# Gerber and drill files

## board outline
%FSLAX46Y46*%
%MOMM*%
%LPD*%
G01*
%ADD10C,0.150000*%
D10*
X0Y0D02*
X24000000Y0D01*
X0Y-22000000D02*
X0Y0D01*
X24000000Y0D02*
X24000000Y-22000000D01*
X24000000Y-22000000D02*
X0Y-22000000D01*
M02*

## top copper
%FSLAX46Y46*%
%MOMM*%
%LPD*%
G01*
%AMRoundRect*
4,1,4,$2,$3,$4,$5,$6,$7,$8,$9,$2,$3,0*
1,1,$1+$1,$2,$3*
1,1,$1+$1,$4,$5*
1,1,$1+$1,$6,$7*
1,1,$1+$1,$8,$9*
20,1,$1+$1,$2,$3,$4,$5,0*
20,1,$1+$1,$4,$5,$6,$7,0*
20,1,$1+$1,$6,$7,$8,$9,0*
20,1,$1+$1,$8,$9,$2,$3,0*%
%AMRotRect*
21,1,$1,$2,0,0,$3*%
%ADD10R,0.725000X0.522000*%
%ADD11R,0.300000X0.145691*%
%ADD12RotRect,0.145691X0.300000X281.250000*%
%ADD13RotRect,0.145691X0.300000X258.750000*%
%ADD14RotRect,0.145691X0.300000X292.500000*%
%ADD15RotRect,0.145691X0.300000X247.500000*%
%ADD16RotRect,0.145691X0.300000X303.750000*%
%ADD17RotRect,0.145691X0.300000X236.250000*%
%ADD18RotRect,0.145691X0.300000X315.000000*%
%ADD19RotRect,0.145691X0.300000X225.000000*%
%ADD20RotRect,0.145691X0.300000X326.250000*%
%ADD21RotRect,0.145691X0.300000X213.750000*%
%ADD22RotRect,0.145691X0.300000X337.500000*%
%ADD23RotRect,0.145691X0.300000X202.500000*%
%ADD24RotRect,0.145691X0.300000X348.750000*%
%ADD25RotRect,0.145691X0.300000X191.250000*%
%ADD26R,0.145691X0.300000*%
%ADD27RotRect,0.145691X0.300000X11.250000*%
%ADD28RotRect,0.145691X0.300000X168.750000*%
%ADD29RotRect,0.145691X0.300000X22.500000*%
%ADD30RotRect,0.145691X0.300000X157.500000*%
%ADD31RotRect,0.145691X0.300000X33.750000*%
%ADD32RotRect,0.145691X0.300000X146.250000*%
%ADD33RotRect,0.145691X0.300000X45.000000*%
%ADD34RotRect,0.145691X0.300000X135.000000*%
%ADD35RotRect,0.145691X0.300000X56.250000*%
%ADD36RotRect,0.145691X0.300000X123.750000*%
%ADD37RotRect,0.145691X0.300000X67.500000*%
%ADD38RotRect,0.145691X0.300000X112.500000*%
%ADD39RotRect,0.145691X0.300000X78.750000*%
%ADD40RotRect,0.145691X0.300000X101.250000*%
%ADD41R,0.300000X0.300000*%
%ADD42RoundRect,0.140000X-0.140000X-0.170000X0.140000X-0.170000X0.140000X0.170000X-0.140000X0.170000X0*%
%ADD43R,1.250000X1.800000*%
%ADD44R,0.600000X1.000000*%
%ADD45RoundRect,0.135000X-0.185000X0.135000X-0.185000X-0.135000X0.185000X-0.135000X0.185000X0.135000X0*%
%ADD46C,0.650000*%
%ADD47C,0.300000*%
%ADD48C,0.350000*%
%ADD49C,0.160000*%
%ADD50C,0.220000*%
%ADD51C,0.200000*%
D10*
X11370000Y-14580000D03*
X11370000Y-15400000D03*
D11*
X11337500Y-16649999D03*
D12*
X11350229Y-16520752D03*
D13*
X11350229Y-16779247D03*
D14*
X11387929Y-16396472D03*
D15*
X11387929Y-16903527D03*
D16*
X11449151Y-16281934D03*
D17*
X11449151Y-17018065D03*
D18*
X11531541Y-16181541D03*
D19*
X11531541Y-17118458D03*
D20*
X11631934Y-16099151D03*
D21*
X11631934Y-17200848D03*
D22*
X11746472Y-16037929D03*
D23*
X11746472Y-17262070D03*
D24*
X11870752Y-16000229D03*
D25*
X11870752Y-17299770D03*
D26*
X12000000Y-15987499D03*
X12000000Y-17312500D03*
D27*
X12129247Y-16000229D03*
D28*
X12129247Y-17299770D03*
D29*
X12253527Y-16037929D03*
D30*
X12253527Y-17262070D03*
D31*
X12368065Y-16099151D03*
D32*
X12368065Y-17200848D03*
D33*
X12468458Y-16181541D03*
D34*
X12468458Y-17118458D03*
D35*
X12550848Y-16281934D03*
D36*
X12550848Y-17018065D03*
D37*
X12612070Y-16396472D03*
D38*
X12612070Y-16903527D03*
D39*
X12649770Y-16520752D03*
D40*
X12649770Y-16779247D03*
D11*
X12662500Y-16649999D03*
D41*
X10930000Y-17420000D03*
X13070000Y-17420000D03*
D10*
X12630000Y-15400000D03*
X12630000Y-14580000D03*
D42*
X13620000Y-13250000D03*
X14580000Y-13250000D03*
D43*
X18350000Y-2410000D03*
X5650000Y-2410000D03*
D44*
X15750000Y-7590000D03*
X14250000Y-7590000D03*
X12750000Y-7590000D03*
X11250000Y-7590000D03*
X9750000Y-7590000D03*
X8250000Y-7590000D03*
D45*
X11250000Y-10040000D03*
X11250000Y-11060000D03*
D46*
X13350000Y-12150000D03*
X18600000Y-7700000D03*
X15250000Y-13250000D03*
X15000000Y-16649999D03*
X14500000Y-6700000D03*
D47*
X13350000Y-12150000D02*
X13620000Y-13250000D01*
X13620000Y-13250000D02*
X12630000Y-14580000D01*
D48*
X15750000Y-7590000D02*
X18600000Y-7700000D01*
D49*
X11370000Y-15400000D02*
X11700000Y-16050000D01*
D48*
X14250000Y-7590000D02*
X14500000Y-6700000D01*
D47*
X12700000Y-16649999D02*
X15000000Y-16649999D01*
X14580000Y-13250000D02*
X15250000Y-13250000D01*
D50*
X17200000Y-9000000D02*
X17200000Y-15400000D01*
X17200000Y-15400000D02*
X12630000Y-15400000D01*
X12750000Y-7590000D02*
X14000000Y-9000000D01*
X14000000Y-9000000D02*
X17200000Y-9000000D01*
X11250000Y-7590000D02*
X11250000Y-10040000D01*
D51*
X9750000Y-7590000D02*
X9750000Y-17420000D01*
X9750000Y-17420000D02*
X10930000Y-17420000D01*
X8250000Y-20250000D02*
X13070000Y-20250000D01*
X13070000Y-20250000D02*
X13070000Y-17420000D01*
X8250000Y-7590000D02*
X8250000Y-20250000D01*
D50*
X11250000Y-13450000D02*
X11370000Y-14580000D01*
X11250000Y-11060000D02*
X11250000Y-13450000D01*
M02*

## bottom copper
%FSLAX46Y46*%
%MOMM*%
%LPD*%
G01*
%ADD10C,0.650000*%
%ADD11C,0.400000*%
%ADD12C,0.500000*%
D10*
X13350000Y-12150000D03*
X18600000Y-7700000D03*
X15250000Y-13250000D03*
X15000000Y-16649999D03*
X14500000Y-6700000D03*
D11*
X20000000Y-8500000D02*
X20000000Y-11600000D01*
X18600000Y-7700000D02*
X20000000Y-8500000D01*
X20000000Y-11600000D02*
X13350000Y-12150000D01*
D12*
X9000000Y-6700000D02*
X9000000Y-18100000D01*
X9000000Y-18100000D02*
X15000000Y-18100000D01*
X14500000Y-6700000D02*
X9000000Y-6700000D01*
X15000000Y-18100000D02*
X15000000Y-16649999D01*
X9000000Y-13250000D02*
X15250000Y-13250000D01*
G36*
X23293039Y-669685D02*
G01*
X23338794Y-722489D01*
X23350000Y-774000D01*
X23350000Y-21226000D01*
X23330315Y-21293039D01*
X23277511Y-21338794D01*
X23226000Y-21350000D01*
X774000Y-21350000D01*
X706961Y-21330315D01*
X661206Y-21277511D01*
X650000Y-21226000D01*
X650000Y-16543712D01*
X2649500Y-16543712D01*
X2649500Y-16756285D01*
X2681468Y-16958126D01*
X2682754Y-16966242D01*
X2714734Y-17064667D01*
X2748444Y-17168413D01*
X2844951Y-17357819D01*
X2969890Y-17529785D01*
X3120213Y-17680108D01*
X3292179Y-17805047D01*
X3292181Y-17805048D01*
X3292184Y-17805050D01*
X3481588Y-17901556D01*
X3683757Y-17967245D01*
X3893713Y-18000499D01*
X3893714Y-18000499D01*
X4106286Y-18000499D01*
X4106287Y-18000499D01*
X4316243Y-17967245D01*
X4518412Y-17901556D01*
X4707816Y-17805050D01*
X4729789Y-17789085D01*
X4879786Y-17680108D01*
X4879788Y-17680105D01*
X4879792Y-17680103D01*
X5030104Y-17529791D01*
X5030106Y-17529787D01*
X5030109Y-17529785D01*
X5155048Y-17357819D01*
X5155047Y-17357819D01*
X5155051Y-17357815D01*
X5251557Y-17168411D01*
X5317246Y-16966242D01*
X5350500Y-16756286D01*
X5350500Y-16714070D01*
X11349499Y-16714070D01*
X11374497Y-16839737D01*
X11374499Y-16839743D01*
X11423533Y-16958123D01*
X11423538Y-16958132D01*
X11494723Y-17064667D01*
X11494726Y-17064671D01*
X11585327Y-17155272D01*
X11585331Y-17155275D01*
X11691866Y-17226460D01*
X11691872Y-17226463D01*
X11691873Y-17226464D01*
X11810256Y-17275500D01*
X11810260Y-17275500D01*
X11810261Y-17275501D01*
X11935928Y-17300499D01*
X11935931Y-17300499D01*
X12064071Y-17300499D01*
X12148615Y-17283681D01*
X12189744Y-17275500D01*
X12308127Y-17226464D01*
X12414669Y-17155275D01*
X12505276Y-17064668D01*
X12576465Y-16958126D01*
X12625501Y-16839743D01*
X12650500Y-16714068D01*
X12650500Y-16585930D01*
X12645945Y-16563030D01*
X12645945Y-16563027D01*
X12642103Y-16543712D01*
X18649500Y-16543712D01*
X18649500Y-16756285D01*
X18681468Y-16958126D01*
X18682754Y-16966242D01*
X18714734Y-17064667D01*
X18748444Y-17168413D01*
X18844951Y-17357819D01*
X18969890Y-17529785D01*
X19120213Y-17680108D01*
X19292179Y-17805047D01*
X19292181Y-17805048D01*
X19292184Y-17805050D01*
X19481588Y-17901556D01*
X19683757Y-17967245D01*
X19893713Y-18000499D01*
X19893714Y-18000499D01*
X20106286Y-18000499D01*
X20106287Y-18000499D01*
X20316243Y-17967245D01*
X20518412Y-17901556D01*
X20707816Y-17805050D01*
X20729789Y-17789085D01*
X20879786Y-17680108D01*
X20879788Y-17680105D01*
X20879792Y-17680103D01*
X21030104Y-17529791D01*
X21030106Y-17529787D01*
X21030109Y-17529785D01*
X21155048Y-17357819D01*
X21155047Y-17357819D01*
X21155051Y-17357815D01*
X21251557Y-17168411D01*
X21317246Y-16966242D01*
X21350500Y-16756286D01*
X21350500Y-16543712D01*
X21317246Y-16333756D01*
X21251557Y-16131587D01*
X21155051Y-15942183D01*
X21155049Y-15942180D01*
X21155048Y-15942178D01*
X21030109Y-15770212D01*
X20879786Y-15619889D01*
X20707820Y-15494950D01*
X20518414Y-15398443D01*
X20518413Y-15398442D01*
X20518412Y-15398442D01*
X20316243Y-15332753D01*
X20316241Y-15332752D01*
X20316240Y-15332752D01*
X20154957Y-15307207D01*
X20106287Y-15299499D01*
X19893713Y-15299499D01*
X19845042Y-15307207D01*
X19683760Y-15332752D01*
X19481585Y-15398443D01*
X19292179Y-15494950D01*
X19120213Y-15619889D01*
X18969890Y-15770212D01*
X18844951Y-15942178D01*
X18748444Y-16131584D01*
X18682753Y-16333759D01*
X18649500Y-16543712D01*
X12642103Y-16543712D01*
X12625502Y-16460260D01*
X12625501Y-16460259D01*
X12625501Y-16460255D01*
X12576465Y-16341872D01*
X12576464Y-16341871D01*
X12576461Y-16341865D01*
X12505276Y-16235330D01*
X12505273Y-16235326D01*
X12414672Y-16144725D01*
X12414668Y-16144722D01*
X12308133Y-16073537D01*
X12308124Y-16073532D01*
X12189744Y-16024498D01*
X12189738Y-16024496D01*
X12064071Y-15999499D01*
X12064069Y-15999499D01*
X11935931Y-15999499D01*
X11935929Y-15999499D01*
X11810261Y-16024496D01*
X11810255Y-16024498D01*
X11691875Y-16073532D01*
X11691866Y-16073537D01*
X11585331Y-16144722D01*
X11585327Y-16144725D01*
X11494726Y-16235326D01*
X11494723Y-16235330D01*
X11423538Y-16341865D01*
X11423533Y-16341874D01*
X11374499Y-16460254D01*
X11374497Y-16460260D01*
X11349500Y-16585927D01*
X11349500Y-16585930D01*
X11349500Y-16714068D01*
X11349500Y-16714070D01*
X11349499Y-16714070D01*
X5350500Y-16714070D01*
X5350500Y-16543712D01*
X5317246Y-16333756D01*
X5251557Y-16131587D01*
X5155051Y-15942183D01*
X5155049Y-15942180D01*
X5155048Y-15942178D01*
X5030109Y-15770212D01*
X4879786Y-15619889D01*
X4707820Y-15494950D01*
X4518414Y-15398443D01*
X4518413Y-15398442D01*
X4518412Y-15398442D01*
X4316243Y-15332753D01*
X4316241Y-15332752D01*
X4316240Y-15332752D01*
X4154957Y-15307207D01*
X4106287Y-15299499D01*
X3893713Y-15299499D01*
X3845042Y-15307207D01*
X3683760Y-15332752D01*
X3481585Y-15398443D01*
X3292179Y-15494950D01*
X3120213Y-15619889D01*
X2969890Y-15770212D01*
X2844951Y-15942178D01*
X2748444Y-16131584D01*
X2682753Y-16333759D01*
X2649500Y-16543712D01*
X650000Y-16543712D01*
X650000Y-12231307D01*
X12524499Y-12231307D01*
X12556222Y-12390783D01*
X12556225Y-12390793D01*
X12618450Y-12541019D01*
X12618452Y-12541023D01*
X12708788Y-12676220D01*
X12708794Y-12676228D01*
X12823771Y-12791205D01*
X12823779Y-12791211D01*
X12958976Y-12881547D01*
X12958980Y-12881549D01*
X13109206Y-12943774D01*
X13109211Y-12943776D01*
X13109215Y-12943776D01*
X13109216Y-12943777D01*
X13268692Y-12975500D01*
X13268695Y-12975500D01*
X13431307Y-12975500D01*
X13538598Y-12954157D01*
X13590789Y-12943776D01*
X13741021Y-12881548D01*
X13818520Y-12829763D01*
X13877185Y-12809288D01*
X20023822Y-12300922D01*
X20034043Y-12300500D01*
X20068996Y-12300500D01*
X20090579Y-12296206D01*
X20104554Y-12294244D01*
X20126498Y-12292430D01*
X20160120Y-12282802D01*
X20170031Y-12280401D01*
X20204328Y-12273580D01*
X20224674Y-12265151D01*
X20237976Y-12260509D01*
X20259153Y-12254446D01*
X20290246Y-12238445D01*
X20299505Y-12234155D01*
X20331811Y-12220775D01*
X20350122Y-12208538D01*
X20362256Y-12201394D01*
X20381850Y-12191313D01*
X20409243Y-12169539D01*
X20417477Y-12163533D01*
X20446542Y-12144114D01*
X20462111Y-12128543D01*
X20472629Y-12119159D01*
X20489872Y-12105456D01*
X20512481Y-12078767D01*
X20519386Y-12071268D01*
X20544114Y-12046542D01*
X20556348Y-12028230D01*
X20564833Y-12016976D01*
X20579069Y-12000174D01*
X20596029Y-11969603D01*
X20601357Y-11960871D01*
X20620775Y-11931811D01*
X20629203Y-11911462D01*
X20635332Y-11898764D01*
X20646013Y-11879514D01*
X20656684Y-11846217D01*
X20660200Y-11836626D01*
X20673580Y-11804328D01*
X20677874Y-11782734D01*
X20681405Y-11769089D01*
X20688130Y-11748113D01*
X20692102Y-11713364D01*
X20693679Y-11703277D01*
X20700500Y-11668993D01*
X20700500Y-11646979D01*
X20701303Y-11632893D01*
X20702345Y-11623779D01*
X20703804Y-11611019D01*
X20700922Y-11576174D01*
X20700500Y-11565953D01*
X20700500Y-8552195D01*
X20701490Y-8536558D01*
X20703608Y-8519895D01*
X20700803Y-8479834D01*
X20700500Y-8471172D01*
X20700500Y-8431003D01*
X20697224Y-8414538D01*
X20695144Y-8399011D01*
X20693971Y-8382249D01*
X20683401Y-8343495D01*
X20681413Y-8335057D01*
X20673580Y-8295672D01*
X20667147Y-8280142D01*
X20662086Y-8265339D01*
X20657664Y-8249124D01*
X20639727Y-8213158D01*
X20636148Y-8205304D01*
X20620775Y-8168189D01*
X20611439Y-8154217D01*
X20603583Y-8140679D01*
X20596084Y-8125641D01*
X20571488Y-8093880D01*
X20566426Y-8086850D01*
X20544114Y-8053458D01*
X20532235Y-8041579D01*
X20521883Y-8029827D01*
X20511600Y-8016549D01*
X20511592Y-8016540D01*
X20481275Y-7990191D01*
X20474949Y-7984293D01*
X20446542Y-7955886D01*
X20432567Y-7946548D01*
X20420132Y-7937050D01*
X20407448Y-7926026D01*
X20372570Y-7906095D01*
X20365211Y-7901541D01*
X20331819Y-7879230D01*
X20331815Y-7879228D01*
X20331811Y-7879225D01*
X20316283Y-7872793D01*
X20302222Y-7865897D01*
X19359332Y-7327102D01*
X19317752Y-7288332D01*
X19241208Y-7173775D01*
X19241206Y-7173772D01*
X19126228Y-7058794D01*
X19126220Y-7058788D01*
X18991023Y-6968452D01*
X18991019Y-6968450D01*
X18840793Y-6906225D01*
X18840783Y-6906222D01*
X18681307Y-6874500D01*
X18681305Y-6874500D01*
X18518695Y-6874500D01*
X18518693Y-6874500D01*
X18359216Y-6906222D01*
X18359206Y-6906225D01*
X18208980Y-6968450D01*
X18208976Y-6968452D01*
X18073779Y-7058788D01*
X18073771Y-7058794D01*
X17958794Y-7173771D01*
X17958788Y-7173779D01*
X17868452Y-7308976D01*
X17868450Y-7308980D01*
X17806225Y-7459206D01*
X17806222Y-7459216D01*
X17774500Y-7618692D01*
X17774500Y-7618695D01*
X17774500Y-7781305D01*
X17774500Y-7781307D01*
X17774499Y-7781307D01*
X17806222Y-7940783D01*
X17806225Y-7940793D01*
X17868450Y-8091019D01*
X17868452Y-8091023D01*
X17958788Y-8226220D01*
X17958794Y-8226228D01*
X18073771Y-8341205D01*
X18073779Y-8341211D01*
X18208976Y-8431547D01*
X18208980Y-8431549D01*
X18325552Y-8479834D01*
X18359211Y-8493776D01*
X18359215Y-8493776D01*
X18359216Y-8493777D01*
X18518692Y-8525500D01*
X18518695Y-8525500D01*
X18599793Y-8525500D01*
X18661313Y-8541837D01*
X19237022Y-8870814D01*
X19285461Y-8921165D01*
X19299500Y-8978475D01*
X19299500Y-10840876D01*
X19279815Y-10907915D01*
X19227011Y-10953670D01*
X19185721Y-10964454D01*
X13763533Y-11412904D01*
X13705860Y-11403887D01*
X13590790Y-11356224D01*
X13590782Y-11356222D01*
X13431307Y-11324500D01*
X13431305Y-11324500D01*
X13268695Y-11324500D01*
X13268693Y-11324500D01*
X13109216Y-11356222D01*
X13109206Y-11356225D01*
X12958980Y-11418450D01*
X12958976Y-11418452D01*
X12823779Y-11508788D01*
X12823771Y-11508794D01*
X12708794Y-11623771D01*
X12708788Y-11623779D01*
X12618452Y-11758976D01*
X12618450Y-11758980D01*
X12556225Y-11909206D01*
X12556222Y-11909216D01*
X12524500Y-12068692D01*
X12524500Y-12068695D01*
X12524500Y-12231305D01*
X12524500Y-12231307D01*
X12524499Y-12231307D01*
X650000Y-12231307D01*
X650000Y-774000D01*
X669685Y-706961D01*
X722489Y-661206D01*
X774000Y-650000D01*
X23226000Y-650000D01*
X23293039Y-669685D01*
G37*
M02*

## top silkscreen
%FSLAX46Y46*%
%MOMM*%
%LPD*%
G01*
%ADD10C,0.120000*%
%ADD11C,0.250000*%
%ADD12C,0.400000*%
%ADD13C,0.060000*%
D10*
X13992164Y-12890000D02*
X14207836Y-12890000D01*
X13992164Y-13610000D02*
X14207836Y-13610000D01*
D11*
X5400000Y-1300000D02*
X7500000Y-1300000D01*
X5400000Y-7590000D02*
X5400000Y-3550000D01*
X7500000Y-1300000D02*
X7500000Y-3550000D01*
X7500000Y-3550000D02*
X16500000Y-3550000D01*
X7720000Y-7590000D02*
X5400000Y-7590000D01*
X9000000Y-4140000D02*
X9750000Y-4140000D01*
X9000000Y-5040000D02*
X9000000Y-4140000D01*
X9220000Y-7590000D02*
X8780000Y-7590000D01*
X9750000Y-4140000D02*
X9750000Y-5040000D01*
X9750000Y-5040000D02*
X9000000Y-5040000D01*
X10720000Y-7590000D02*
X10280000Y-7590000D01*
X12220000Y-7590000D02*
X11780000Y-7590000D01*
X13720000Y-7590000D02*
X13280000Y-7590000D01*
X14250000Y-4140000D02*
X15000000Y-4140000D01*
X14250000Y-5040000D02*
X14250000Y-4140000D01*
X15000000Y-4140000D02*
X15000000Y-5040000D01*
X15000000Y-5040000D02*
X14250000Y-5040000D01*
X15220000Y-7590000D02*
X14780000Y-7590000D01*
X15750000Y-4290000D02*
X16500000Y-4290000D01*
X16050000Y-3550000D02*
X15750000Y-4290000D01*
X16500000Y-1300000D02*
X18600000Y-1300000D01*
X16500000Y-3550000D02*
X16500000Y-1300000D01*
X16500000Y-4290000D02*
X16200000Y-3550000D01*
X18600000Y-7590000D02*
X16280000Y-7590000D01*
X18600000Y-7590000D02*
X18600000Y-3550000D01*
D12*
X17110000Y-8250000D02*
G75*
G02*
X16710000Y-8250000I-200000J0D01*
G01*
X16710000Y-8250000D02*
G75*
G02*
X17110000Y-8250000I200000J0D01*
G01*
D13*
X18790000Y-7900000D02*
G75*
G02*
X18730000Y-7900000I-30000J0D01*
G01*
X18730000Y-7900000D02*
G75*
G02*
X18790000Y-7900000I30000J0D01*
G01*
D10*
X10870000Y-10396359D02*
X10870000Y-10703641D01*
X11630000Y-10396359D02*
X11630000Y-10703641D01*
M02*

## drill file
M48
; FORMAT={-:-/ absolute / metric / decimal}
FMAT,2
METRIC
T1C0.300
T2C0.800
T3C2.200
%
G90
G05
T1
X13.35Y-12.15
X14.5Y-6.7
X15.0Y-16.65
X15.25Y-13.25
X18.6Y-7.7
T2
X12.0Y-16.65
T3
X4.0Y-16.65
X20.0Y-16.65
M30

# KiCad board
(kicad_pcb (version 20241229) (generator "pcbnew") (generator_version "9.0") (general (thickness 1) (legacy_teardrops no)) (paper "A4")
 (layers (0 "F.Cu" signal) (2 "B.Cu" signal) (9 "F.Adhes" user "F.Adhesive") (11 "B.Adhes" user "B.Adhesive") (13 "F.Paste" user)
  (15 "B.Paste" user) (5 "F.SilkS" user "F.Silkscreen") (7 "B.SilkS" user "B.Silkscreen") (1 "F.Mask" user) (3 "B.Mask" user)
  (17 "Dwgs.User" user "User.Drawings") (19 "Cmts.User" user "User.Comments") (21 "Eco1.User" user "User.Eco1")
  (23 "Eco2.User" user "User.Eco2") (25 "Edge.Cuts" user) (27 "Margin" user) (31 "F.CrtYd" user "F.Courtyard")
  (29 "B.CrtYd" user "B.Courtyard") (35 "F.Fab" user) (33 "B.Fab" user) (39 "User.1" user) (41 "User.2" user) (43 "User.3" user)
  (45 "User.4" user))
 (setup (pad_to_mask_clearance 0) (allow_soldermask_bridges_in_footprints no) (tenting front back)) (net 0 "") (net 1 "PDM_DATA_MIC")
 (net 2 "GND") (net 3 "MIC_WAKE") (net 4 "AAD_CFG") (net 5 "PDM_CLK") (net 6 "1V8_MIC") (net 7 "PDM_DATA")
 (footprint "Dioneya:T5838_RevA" (layer "F.Cu") (at 12 16)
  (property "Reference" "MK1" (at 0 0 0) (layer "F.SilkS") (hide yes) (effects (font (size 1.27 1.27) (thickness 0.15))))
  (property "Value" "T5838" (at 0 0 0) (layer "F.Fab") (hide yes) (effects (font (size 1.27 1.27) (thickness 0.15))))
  (pad "" np_thru_hole circle (at 0 0.649999) (size 0.8 0.8) (drill 0.8) (layers "*.Cu" "*.Mask"))
  (pad "1" smd rect (at -0.63 -1.42 90) (size 0.522 0.725) (layers "F.Cu" "F.Mask" "F.Paste") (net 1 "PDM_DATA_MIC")
   (solder_paste_margin -0.05) (thermal_bridge_angle 45))
  (pad "2" smd rect (at -0.63 -0.6 90) (size 0.522 0.725) (layers "F.Cu" "F.Mask" "F.Paste") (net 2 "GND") (solder_paste_margin -0.05)
   (thermal_bridge_angle 45))
  (pad "3" smd rect (at -0.6625 0.649999 270) (size 0.145691 0.3) (layers "F.Cu" "F.Mask") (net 2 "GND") (thermal_bridge_angle 45))
  (pad "3" smd rect (at -0.649771 0.520752 281.25) (size 0.145691 0.3) (layers "F.Cu" "F.Mask") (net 2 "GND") (thermal_bridge_angle 45))
  (pad "3" smd rect (at -0.649771 0.779247 258.75) (size 0.145691 0.3) (layers "F.Cu" "F.Mask") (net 2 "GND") (thermal_bridge_angle 45))
  (pad "3" smd rect (at -0.612071 0.396472 292.5) (size 0.145691 0.3) (layers "F.Cu" "F.Mask") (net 2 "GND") (thermal_bridge_angle 45))
  (pad "3" smd rect (at -0.612071 0.903527 247.5) (size 0.145691 0.3) (layers "F.Cu" "F.Mask") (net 2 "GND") (thermal_bridge_angle 45))
  (pad "3" smd rect (at -0.550849 0.281934 303.75) (size 0.145691 0.3) (layers "F.Cu" "F.Mask") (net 2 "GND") (thermal_bridge_angle 45))
  (pad "3" smd rect (at -0.550849 1.018065 236.25) (size 0.145691 0.3) (layers "F.Cu" "F.Mask") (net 2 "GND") (thermal_bridge_angle 45))
  (pad "3" smd rect (at -0.468459 0.181541 315) (size 0.145691 0.3) (layers "F.Cu" "F.Mask") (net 2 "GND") (thermal_bridge_angle 45))
  (pad "3" smd rect (at -0.468459 1.118458 225) (size 0.145691 0.3) (layers "F.Cu" "F.Mask") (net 2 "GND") (thermal_bridge_angle 45))
  (pad "3" smd rect (at -0.368066 0.099151 326.25) (size 0.145691 0.3) (layers "F.Cu" "F.Mask") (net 2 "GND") (thermal_bridge_angle 45))
  (pad "3" smd rect (at -0.368066 1.200848 213.75) (size 0.145691 0.3) (layers "F.Cu" "F.Mask") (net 2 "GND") (thermal_bridge_angle 45))
  (pad "3" smd rect (at -0.253528 0.037929 337.5) (size 0.145691 0.3) (layers "F.Cu" "F.Mask") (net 2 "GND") (thermal_bridge_angle 45))
  (pad "3" smd rect (at -0.253528 1.26207 202.5) (size 0.145691 0.3) (layers "F.Cu" "F.Mask") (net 2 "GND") (thermal_bridge_angle 45))
  (pad "3" smd rect (at -0.129248 0.000229 348.75) (size 0.145691 0.3) (layers "F.Cu" "F.Mask") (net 2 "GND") (thermal_bridge_angle 45))
  (pad "3" smd rect (at -0.129248 1.29977 191.25) (size 0.145691 0.3) (layers "F.Cu" "F.Mask") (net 2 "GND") (thermal_bridge_angle 45))
  (pad "3" smd rect (at 0 -0.012501) (size 0.145691 0.3) (layers "F.Cu" "F.Mask") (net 2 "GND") (thermal_bridge_angle 45))
  (pad "3" smd rect (at 0 1.3125 180) (size 0.145691 0.3) (layers "F.Cu" "F.Mask") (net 2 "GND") (thermal_bridge_angle 45))
  (pad "3" smd rect (at 0.129247 0.000229 11.25) (size 0.145691 0.3) (layers "F.Cu" "F.Mask") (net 2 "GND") (thermal_bridge_angle 45))
  (pad "3" smd rect (at 0.129247 1.29977 168.75) (size 0.145691 0.3) (layers "F.Cu" "F.Mask") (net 2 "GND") (thermal_bridge_angle 45))
  (pad "3" smd rect (at 0.253527 0.037929 22.5) (size 0.145691 0.3) (layers "F.Cu" "F.Mask") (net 2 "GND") (thermal_bridge_angle 45))
  (pad "3" smd rect (at 0.253527 1.26207 157.5) (size 0.145691 0.3) (layers "F.Cu" "F.Mask") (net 2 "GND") (thermal_bridge_angle 45))
  (pad "3" smd rect (at 0.368065 0.099151 33.75) (size 0.145691 0.3) (layers "F.Cu" "F.Mask") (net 2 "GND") (thermal_bridge_angle 45))
  (pad "3" smd rect (at 0.368065 1.200848 146.25) (size 0.145691 0.3) (layers "F.Cu" "F.Mask") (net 2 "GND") (thermal_bridge_angle 45))
  (pad "3" smd rect (at 0.468458 0.181541 45) (size 0.145691 0.3) (layers "F.Cu" "F.Mask") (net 2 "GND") (thermal_bridge_angle 45))
  (pad "3" smd rect (at 0.468458 1.118458 135) (size 0.145691 0.3) (layers "F.Cu" "F.Mask") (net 2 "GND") (thermal_bridge_angle 45))
  (pad "3" smd rect (at 0.550848 0.281934 56.25) (size 0.145691 0.3) (layers "F.Cu" "F.Mask") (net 2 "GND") (thermal_bridge_angle 45))
  (pad "3" smd rect (at 0.550848 1.018065 123.75) (size 0.145691 0.3) (layers "F.Cu" "F.Mask") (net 2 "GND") (thermal_bridge_angle 45))
  (pad "3" smd rect (at 0.61207 0.396472 67.5) (size 0.145691 0.3) (layers "F.Cu" "F.Mask") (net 2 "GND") (thermal_bridge_angle 45))
  (pad "3" smd rect (at 0.61207 0.903527 112.5) (size 0.145691 0.3) (layers "F.Cu" "F.Mask") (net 2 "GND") (thermal_bridge_angle 45))
  (pad "3" smd rect (at 0.64977 0.520752 78.75) (size 0.145691 0.3) (layers "F.Cu" "F.Mask") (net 2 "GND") (thermal_bridge_angle 45))
  (pad "3" smd rect (at 0.64977 0.779247 101.25) (size 0.145691 0.3) (layers "F.Cu" "F.Mask") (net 2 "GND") (thermal_bridge_angle 45))
  (pad "3" smd rect (at 0.6625 0.649999 90) (size 0.145691 0.3) (layers "F.Cu" "F.Mask") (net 2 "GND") (thermal_bridge_angle 45))
  (pad "4" smd rect (at -1.07 1.42 90) (size 0.3 0.3) (layers "F.Cu" "F.Mask" "F.Paste") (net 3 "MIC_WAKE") (solder_paste_margin -0.015)
   (thermal_bridge_angle 45))
  (pad "5" smd rect (at 1.07 1.42 90) (size 0.3 0.3) (layers "F.Cu" "F.Mask" "F.Paste") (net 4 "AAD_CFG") (solder_paste_margin -0.015)
   (thermal_bridge_angle 45))
  (pad "6" smd rect (at 0.63 -0.6 90) (size 0.522 0.725) (layers "F.Cu" "F.Mask" "F.Paste") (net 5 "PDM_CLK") (solder_paste_margin -0.05)
   (thermal_bridge_angle 45))
  (pad "7" smd rect (at 0.63 -1.42 90) (size 0.522 0.725) (layers "F.Cu" "F.Mask" "F.Paste") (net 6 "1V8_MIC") (solder_paste_margin -0.05)
   (thermal_bridge_angle 45)))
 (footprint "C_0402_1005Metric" (layer "F.Cu") (at 14.1 13.25)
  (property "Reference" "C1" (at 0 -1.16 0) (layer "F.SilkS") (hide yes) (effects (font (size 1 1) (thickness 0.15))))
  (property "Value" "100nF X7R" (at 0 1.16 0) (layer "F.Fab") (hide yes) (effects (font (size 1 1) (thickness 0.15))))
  (fp_line (start -0.107836 -0.36) (end 0.107836 -0.36) (stroke (width 0.12) (type solid)) (layer "F.SilkS"))
  (fp_line (start -0.107836 0.36) (end 0.107836 0.36) (stroke (width 0.12) (type solid)) (layer "F.SilkS"))
  (pad "1" smd roundrect (at -0.48 0) (size 0.56 0.62) (layers "F.Cu" "F.Mask" "F.Paste") (roundrect_rratio 0.25) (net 6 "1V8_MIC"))
  (pad "2" smd roundrect (at 0.48 0) (size 0.56 0.62) (layers "F.Cu" "F.Mask" "F.Paste") (roundrect_rratio 0.25) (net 2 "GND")))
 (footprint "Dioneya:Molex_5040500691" (layer "F.Cu") (at 12 5 180)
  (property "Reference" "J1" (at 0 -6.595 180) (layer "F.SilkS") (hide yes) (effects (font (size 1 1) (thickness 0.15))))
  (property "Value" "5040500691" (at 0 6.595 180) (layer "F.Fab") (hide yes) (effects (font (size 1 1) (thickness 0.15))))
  (fp_line (start 6.6 3.7) (end 4.5 3.7) (stroke (width 0.25) (type solid)) (layer "F.SilkS"))
  (fp_line (start 6.6 -2.59) (end 6.6 1.45) (stroke (width 0.25) (type solid)) (layer "F.SilkS"))
  (fp_line (start 4.5 3.7) (end 4.5 1.45) (stroke (width 0.25) (type solid)) (layer "F.SilkS"))
  (fp_line (start 4.5 1.45) (end -4.5 1.45) (stroke (width 0.25) (type solid)) (layer "F.SilkS"))
  (fp_line (start 4.28 -2.59) (end 6.6 -2.59) (stroke (width 0.25) (type solid)) (layer "F.SilkS"))
  (fp_line (start 3 0.86) (end 2.25 0.86) (stroke (width 0.25) (type solid)) (layer "F.SilkS"))
  (fp_line (start 3 -0.04) (end 3 0.86) (stroke (width 0.25) (type solid)) (layer "F.SilkS"))
  (fp_line (start 2.78 -2.59) (end 3.22 -2.59) (stroke (width 0.25) (type solid)) (layer "F.SilkS"))
  (fp_line (start 2.25 0.86) (end 2.25 -0.04) (stroke (width 0.25) (type solid)) (layer "F.SilkS"))
  (fp_line (start 2.25 -0.04) (end 3 -0.04) (stroke (width 0.25) (type solid)) (layer "F.SilkS"))
  (fp_line (start 1.28 -2.59) (end 1.72 -2.59) (stroke (width 0.25) (type solid)) (layer "F.SilkS"))
  (fp_line (start -0.22 -2.59) (end 0.22 -2.59) (stroke (width 0.25) (type solid)) (layer "F.SilkS"))
  (fp_line (start -1.72 -2.59) (end -1.28 -2.59) (stroke (width 0.25) (type solid)) (layer "F.SilkS"))
  (fp_line (start -2.25 0.86) (end -3 0.86) (stroke (width 0.25) (type solid)) (layer "F.SilkS"))
  (fp_line (start -2.25 -0.04) (end -2.25 0.86) (stroke (width 0.25) (type solid)) (layer "F.SilkS"))
  (fp_line (start -3 0.86) (end -3 -0.04) (stroke (width 0.25) (type solid)) (layer "F.SilkS"))
  (fp_line (start -3 -0.04) (end -2.25 -0.04) (stroke (width 0.25) (type solid)) (layer "F.SilkS"))
  (fp_line (start -3.22 -2.59) (end -2.78 -2.59) (stroke (width 0.25) (type solid)) (layer "F.SilkS"))
  (fp_line (start -3.75 0.71) (end -4.5 0.71) (stroke (width 0.25) (type solid)) (layer "F.SilkS"))
  (fp_line (start -4.05 1.45) (end -3.75 0.71) (stroke (width 0.25) (type solid)) (layer "F.SilkS"))
  (fp_line (start -4.5 3.7) (end -6.6 3.7) (stroke (width 0.25) (type solid)) (layer "F.SilkS"))
  (fp_line (start -4.5 1.45) (end -4.5 3.7) (stroke (width 0.25) (type solid)) (layer "F.SilkS"))
  (fp_line (start -4.5 0.71) (end -4.2 1.45) (stroke (width 0.25) (type solid)) (layer "F.SilkS"))
  (fp_line (start -6.6 -2.59) (end -4.28 -2.59) (stroke (width 0.25) (type solid)) (layer "F.SilkS"))
  (fp_line (start -6.6 -2.59) (end -6.6 1.45) (stroke (width 0.25) (type solid)) (layer "F.SilkS"))
  (fp_circle (center -4.91 -3.25) (end -4.71 -3.25) (stroke (width 0.4) (type solid)) (fill no) (layer "F.SilkS"))
  (fp_circle (center -6.76 -2.9) (end -6.73 -2.9) (stroke (width 0.06) (type solid)) (fill no) (layer "F.SilkS"))
  (pad "" smd rect (at -6.35 2.59) (size 1.25 1.8) (layers "F.Cu" "F.Mask" "F.Paste"))
  (pad "" smd rect (at 6.35 2.59) (size 1.25 1.8) (layers "F.Cu" "F.Mask" "F.Paste"))
  (pad "1" smd rect (at -3.75 -2.59) (size 0.6 1) (layers "F.Cu" "F.Mask" "F.Paste") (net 6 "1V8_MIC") (solder_paste_margin 0))
  (pad "2" smd rect (at -2.25 -2.59) (size 0.6 1) (layers "F.Cu" "F.Mask" "F.Paste") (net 2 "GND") (solder_paste_margin 0))
  (pad "3" smd rect (at -0.75 -2.59) (size 0.6 1) (layers "F.Cu" "F.Mask" "F.Paste") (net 5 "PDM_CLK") (solder_paste_margin 0))
  (pad "4" smd rect (at 0.75 -2.59) (size 0.6 1) (layers "F.Cu" "F.Mask" "F.Paste") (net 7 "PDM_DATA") (solder_paste_margin 0))
  (pad "5" smd rect (at 2.25 -2.59) (size 0.6 1) (layers "F.Cu" "F.Mask" "F.Paste") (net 3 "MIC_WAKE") (solder_paste_margin 0))
  (pad "6" smd rect (at 3.75 -2.59) (size 0.6 1) (layers "F.Cu" "F.Mask" "F.Paste") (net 4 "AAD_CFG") (solder_paste_margin 0)))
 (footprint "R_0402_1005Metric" (layer "F.Cu") (at 11.25 10.55 -90)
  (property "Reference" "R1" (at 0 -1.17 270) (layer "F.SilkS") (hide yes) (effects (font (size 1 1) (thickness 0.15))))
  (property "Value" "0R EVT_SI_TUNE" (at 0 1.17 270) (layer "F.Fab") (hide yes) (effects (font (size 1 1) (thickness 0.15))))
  (fp_line (start -0.153641 0.38) (end 0.153641 0.38) (stroke (width 0.12) (type solid)) (layer "F.SilkS"))
  (fp_line (start -0.153641 -0.38) (end 0.153641 -0.38) (stroke (width 0.12) (type solid)) (layer "F.SilkS"))
  (pad "1" smd roundrect (at -0.51 0 270) (size 0.54 0.64) (layers "F.Cu" "F.Mask" "F.Paste") (roundrect_rratio 0.25) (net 7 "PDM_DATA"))
  (pad "2" smd roundrect (at 0.51 0 270) (size 0.54 0.64) (layers "F.Cu" "F.Mask" "F.Paste") (roundrect_rratio 0.25) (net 1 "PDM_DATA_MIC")))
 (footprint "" (layer "F.Cu") (at 4 16.649999)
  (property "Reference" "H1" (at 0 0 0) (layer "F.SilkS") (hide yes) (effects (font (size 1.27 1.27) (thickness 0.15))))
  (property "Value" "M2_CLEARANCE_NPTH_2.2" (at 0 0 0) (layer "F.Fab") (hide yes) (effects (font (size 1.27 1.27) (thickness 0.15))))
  (pad "" np_thru_hole circle (at 0 0) (size 2.2 2.2) (drill 2.2) (layers "*.Cu" "*.Mask")))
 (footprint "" (layer "F.Cu") (at 20 16.649999)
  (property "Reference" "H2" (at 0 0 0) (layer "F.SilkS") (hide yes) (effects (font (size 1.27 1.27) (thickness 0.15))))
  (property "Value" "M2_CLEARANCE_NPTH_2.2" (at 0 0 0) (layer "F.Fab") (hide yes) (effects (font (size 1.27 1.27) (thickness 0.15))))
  (pad "" np_thru_hole circle (at 0 0) (size 2.2 2.2) (drill 2.2) (layers "*.Cu" "*.Mask")))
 (gr_line (start 0 0) (end 24 0) (stroke (width 0.15) (type default)) (layer "Edge.Cuts"))
 (gr_line (start 0 22) (end 0 0) (stroke (width 0.15) (type default)) (layer "Edge.Cuts"))
 (gr_line (start 24 0) (end 24 22) (stroke (width 0.15) (type default)) (layer "Edge.Cuts"))
 (gr_line (start 24 22) (end 0 22) (stroke (width 0.15) (type default)) (layer "Edge.Cuts"))
 (segment (start 13.35 12.15) (end 13.62 13.25) (width 0.3) (layer "F.Cu") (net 6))
 (segment (start 13.62 13.25) (end 12.63 14.58) (width 0.3) (layer "F.Cu") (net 6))
 (segment (start 15.75 7.59) (end 18.6 7.7) (width 0.35) (layer "F.Cu") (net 6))
 (via (at 13.35 12.15) (size 0.65) (drill 0.3) (layers "F.Cu" "B.Cu") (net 6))
 (via (at 18.6 7.7) (size 0.65) (drill 0.3) (layers "F.Cu" "B.Cu") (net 6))
 (segment (start 20 8.5) (end 20 11.6) (width 0.4) (layer "B.Cu") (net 6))
 (segment (start 18.6 7.7) (end 20 8.5) (width 0.4) (layer "B.Cu") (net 6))
 (segment (start 20 11.6) (end 13.35 12.15) (width 0.4) (layer "B.Cu") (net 6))
 (segment (start 11.37 15.4) (end 11.7 16.05) (width 0.16) (layer "F.Cu") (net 2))
 (segment (start 14.25 7.59) (end 14.5 6.7) (width 0.35) (layer "F.Cu") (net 2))
 (segment (start 12.7 16.649999) (end 15 16.649999) (width 0.3) (layer "F.Cu") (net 2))
 (segment (start 14.58 13.25) (end 15.25 13.25) (width 0.3) (layer "F.Cu") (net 2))
 (via (at 15.25 13.25) (size 0.65) (drill 0.3) (layers "F.Cu" "B.Cu") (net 2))
 (via (at 15 16.649999) (size 0.65) (drill 0.3) (layers "F.Cu" "B.Cu") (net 2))
 (via (at 14.5 6.7) (size 0.65) (drill 0.3) (layers "F.Cu" "B.Cu") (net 2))
 (segment (start 9 6.7) (end 9 18.1) (width 0.5) (layer "B.Cu") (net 2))
 (segment (start 9 18.1) (end 15 18.1) (width 0.5) (layer "B.Cu") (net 2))
 (segment (start 14.5 6.7) (end 9 6.7) (width 0.5) (layer "B.Cu") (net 2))
 (segment (start 15 18.1) (end 15 16.649999) (width 0.5) (layer "B.Cu") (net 2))
 (segment (start 9 13.25) (end 15.25 13.25) (width 0.5) (layer "B.Cu") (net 2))
 (segment (start 17.2 9) (end 17.2 15.4) (width 0.22) (layer "F.Cu") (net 5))
 (segment (start 17.2 15.4) (end 12.63 15.4) (width 0.22) (layer "F.Cu") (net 5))
 (segment (start 12.75 7.59) (end 14 9) (width 0.22) (layer "F.Cu") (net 5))
 (segment (start 14 9) (end 17.2 9) (width 0.22) (layer "F.Cu") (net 5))
 (segment (start 11.25 7.59) (end 11.25 10.04) (width 0.22) (layer "F.Cu") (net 7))
 (segment (start 9.75 7.59) (end 9.75 17.42) (width 0.2) (layer "F.Cu") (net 3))
 (segment (start 9.75 17.42) (end 10.93 17.42) (width 0.2) (layer "F.Cu") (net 3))
 (segment (start 8.25 20.25) (end 13.07 20.25) (width 0.2) (layer "F.Cu") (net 4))
 (segment (start 13.07 20.25) (end 13.07 17.42) (width 0.2) (layer "F.Cu") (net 4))
 (segment (start 8.25 7.59) (end 8.25 20.25) (width 0.2) (layer "F.Cu") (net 4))
 (segment (start 11.25 13.45) (end 11.37 14.58) (width 0.22) (layer "F.Cu") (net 1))
 (segment (start 11.25 11.06) (end 11.25 13.45) (width 0.22) (layer "F.Cu") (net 1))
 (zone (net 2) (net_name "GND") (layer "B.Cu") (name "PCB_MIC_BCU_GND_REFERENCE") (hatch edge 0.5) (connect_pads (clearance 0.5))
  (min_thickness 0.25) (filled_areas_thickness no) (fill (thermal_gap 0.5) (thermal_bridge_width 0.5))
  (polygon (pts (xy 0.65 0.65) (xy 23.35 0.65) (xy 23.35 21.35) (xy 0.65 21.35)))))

